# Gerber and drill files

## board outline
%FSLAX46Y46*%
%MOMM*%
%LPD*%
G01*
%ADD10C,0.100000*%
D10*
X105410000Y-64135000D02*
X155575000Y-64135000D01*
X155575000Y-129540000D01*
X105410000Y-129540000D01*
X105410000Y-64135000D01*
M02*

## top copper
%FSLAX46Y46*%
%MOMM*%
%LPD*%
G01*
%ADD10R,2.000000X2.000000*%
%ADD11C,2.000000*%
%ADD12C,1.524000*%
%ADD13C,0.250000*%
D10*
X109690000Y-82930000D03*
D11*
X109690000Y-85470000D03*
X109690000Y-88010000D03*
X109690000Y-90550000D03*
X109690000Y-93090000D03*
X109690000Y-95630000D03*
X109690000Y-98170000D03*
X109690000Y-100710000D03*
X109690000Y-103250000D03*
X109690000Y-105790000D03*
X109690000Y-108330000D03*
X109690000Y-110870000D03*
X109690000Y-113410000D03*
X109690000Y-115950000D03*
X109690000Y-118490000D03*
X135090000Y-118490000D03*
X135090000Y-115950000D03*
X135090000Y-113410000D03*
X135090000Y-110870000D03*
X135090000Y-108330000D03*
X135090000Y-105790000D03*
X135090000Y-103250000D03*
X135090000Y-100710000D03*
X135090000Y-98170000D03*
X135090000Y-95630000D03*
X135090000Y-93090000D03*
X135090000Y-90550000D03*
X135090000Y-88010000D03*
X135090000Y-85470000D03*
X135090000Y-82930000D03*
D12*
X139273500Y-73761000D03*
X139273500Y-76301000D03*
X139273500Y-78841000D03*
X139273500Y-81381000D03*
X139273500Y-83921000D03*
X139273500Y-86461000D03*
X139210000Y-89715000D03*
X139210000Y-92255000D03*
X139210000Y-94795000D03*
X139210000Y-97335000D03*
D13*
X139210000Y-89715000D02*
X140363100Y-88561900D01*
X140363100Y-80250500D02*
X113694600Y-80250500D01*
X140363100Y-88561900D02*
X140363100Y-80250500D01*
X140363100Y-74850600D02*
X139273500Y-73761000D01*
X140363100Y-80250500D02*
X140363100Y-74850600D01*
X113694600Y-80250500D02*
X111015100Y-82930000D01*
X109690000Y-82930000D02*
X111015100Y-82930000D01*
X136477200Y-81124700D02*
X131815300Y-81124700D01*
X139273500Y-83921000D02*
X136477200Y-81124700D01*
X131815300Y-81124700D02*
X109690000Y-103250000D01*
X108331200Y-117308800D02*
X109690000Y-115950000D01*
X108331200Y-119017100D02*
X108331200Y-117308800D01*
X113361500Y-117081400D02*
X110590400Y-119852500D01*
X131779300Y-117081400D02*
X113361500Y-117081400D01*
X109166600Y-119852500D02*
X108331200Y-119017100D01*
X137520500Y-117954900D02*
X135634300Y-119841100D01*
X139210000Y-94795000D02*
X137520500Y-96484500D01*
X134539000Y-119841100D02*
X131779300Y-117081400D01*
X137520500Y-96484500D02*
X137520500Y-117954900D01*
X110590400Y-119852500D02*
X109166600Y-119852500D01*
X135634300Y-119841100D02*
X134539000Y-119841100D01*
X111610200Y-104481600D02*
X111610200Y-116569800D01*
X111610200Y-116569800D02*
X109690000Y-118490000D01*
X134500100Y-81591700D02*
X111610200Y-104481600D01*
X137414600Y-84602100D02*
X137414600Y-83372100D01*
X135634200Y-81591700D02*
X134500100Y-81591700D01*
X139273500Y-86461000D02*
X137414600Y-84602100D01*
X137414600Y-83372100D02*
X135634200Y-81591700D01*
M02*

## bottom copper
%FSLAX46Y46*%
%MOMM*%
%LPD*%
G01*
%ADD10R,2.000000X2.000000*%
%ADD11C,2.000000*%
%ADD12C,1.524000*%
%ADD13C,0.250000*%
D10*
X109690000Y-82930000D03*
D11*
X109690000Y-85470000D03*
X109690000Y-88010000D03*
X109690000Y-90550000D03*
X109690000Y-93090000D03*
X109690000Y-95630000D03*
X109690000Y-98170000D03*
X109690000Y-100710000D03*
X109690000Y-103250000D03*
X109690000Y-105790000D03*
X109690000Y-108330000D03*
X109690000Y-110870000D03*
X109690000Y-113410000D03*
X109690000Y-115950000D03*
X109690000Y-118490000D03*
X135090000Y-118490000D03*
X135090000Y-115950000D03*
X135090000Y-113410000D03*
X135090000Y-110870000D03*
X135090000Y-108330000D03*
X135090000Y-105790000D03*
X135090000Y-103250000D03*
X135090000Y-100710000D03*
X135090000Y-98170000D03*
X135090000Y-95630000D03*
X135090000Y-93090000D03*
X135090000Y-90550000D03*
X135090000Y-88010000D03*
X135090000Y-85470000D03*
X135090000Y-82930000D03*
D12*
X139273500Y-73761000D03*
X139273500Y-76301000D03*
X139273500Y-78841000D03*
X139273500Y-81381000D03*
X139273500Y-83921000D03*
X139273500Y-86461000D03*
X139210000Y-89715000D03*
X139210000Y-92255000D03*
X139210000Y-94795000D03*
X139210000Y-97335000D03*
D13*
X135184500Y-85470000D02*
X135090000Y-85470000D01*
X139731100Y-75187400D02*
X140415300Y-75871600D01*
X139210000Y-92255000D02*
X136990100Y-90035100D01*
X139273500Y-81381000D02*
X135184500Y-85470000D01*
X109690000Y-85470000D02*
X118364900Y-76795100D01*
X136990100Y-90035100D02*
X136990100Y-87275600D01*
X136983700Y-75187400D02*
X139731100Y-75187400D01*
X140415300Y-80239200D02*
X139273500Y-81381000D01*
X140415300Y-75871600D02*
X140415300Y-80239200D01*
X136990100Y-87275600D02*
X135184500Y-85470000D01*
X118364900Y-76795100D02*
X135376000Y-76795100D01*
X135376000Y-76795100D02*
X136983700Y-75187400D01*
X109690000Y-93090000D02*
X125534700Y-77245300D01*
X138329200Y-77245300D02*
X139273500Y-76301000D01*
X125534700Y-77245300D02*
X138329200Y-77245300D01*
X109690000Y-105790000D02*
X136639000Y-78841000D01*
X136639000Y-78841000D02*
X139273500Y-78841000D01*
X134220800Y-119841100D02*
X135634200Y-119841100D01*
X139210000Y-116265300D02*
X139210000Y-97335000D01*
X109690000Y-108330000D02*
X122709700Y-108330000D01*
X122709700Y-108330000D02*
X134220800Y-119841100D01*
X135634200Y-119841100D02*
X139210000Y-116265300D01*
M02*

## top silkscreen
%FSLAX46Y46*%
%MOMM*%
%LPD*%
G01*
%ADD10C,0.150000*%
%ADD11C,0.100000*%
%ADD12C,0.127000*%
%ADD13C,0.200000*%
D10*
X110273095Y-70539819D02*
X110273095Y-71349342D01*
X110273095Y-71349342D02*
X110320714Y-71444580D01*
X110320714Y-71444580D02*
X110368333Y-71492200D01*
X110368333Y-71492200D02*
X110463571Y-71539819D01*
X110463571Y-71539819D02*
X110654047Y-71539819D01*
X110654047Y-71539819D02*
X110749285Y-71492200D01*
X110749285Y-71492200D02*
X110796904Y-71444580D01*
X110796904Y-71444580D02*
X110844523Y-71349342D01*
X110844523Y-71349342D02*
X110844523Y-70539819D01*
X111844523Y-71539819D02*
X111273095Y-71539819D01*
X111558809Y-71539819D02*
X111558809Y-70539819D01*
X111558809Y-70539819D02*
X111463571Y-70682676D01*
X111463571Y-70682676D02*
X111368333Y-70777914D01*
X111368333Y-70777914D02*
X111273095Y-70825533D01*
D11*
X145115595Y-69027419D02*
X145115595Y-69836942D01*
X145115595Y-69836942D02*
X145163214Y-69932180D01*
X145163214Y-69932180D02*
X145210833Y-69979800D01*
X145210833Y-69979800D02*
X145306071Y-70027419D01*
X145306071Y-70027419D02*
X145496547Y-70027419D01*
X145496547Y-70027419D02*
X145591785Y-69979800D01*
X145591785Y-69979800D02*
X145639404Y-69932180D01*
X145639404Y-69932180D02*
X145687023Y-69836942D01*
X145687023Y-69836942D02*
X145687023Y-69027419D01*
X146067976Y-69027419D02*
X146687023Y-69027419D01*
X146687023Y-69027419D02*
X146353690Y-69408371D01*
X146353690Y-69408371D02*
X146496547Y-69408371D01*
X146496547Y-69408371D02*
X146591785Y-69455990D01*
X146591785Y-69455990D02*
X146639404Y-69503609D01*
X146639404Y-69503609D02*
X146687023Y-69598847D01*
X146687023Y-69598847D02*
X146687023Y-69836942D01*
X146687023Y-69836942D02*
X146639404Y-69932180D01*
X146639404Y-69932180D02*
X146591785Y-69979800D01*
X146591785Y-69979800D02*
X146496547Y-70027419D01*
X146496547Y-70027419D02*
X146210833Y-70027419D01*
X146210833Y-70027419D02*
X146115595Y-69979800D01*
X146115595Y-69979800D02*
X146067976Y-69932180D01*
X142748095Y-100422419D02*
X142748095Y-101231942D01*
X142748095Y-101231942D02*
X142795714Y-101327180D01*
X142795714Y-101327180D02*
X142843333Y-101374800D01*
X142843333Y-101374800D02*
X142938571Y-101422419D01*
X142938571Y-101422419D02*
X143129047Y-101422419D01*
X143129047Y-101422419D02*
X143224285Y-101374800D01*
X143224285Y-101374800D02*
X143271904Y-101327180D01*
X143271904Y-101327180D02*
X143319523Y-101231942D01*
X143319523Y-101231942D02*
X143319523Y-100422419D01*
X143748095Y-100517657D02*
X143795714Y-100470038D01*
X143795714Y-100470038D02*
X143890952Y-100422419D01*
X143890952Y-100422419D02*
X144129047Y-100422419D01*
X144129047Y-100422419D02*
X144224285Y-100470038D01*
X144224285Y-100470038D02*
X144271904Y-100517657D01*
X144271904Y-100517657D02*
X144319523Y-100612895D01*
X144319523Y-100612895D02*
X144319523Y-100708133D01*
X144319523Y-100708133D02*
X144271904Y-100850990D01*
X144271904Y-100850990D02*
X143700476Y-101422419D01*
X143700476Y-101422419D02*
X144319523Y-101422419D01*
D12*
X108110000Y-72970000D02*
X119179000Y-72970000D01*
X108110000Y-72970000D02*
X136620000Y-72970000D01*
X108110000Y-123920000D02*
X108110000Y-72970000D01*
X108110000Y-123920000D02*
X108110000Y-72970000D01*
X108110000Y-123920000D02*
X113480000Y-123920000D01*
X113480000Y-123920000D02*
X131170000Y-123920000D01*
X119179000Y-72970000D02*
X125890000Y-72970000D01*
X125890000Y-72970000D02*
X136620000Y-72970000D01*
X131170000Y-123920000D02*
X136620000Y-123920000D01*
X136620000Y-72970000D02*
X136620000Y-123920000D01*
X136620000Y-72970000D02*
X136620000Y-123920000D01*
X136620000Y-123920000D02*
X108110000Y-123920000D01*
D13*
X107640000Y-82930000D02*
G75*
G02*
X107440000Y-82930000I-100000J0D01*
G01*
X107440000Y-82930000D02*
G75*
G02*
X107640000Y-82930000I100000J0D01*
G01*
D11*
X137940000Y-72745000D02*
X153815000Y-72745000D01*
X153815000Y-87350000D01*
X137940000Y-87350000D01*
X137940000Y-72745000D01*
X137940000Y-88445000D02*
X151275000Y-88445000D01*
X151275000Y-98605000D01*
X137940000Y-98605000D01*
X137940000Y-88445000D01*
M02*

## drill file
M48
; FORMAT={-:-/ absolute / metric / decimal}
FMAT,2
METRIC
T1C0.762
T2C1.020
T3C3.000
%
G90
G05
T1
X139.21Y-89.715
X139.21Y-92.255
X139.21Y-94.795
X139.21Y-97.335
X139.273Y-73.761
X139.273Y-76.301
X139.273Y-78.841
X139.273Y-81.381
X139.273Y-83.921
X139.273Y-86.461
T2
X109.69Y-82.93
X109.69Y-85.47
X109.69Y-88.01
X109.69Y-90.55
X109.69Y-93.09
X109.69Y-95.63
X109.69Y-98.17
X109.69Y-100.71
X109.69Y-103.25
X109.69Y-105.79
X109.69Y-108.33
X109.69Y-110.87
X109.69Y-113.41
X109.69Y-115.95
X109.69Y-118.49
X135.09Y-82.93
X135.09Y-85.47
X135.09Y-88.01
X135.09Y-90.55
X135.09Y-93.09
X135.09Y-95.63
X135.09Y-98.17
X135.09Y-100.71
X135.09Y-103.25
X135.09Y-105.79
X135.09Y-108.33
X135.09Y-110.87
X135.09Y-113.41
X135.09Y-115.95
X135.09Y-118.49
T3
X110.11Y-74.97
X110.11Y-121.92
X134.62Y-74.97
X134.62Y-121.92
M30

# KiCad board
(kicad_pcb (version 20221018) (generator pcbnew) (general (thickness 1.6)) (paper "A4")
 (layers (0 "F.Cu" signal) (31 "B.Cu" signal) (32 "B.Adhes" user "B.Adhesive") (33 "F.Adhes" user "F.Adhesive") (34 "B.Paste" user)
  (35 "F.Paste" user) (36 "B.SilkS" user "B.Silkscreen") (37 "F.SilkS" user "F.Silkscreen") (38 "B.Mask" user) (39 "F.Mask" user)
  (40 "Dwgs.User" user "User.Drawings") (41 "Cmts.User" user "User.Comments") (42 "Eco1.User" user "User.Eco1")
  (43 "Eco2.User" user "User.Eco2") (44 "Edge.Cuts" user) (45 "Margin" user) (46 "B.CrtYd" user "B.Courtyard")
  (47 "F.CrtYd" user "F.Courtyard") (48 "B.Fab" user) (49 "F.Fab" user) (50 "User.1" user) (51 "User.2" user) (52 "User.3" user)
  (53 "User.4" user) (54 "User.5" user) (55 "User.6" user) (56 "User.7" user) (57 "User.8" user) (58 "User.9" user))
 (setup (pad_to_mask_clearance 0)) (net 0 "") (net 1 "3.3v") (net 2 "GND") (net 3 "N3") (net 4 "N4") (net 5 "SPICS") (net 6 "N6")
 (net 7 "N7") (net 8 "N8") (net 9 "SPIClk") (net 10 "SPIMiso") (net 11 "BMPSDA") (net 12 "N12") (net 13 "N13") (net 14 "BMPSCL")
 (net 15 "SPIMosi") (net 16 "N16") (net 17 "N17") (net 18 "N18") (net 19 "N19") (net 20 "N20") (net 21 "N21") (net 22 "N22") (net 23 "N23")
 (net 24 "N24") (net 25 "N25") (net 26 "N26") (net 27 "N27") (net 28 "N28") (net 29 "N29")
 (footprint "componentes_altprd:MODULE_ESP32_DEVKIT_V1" (layer "F.Cu") (at 122.39 98.445)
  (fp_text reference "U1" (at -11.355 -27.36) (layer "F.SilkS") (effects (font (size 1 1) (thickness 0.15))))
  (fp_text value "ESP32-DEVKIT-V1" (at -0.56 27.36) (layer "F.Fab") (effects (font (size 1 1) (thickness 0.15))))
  (fp_line (start -14.28 -25.475) (end -3.211 -25.475) (stroke (width 0.127) (type solid)) (layer "F.SilkS"))
  (fp_line (start -14.28 -25.475) (end 14.23 -25.475) (stroke (width 0.127) (type solid)) (layer "F.SilkS"))
  (fp_line (start -14.28 25.475) (end -14.28 -25.475) (stroke (width 0.127) (type solid)) (layer "F.SilkS"))
  (fp_line (start -14.28 25.475) (end -14.28 -25.475) (stroke (width 0.127) (type solid)) (layer "F.SilkS"))
  (fp_line (start -14.28 25.475) (end -8.91 25.475) (stroke (width 0.127) (type solid)) (layer "F.SilkS"))
  (fp_line (start -8.91 25.475) (end 8.78 25.475) (stroke (width 0.127) (type solid)) (layer "F.SilkS"))
  (fp_line (start -3.211 -25.475) (end 3.5 -25.475) (stroke (width 0.127) (type solid)) (layer "F.SilkS"))
  (fp_line (start 3.5 -25.475) (end 14.23 -25.475) (stroke (width 0.127) (type solid)) (layer "F.SilkS"))
  (fp_line (start 8.78 25.475) (end 14.23 25.475) (stroke (width 0.127) (type solid)) (layer "F.SilkS"))
  (fp_line (start 14.23 -25.475) (end 14.23 25.475) (stroke (width 0.127) (type solid)) (layer "F.SilkS"))
  (fp_line (start 14.23 -25.475) (end 14.23 25.475) (stroke (width 0.127) (type solid)) (layer "F.SilkS"))
  (fp_line (start 14.23 25.475) (end -14.28 25.475) (stroke (width 0.127) (type solid)) (layer "F.SilkS"))
  (fp_circle (center -14.85 -15.515) (end -14.75 -15.515) (stroke (width 0.2) (type solid)) (fill none) (layer "F.SilkS"))
  (pad "" np_thru_hole circle (at -12.28 -23.475) (size 3 3) (drill 3) (layers "*.Cu" "*.Mask"))
  (pad "" np_thru_hole circle (at -12.28 23.475) (size 3 3) (drill 3) (layers "*.Cu" "*.Mask"))
  (pad "" np_thru_hole circle (at 12.23 -23.475) (size 3 3) (drill 3) (layers "*.Cu" "*.Mask"))
  (pad "" np_thru_hole circle (at 12.23 23.475) (size 3 3) (drill 3) (layers "*.Cu" "*.Mask"))
  (pad "1" thru_hole rect (at -12.7 -15.515) (size 2 2) (drill 1.02) (layers "*.Cu" "*.Mask") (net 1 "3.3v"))
  (pad "2" thru_hole circle (at -12.7 -12.975) (size 2 2) (drill 1.02) (layers "*.Cu" "*.Mask") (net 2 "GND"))
  (pad "3" thru_hole circle (at -12.7 -10.435) (size 2 2) (drill 1.02) (layers "*.Cu" "*.Mask") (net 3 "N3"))
  (pad "4" thru_hole circle (at -12.7 -7.895) (size 2 2) (drill 1.02) (layers "*.Cu" "*.Mask") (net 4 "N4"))
  (pad "5" thru_hole circle (at -12.7 -5.355) (size 2 2) (drill 1.02) (layers "*.Cu" "*.Mask") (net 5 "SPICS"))
  (pad "6" thru_hole circle (at -12.7 -2.815) (size 2 2) (drill 1.02) (layers "*.Cu" "*.Mask") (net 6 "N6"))
  (pad "7" thru_hole circle (at -12.7 -0.275) (size 2 2) (drill 1.02) (layers "*.Cu" "*.Mask") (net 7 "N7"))
  (pad "8" thru_hole circle (at -12.7 2.265) (size 2 2) (drill 1.02) (layers "*.Cu" "*.Mask") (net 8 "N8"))
  (pad "9" thru_hole circle (at -12.7 4.805) (size 2 2) (drill 1.02) (layers "*.Cu" "*.Mask") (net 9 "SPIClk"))
  (pad "10" thru_hole circle (at -12.7 7.345) (size 2 2) (drill 1.02) (layers "*.Cu" "*.Mask") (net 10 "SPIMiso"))
  (pad "11" thru_hole circle (at -12.7 9.885) (size 2 2) (drill 1.02) (layers "*.Cu" "*.Mask") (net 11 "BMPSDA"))
  (pad "12" thru_hole circle (at -12.7 12.425) (size 2 2) (drill 1.02) (layers "*.Cu" "*.Mask") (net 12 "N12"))
  (pad "13" thru_hole circle (at -12.7 14.965) (size 2 2) (drill 1.02) (layers "*.Cu" "*.Mask") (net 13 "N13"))
  (pad "14" thru_hole circle (at -12.7 17.505) (size 2 2) (drill 1.02) (layers "*.Cu" "*.Mask") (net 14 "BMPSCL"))
  (pad "15" thru_hole circle (at -12.7 20.045) (size 2 2) (drill 1.02) (layers "*.Cu" "*.Mask") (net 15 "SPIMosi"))
  (pad "16" thru_hole circle (at 12.7 20.045) (size 2 2) (drill 1.02) (layers "*.Cu" "*.Mask") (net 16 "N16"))
  (pad "17" thru_hole circle (at 12.7 17.505) (size 2 2) (drill 1.02) (layers "*.Cu" "*.Mask") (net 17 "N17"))
  (pad "18" thru_hole circle (at 12.7 14.965) (size 2 2) (drill 1.02) (layers "*.Cu" "*.Mask") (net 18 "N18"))
  (pad "19" thru_hole circle (at 12.7 12.425) (size 2 2) (drill 1.02) (layers "*.Cu" "*.Mask") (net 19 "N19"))
  (pad "20" thru_hole circle (at 12.7 9.885) (size 2 2) (drill 1.02) (layers "*.Cu" "*.Mask") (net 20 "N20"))
  (pad "21" thru_hole circle (at 12.7 7.345) (size 2 2) (drill 1.02) (layers "*.Cu" "*.Mask") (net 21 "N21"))
  (pad "22" thru_hole circle (at 12.7 4.805) (size 2 2) (drill 1.02) (layers "*.Cu" "*.Mask") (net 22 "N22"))
  (pad "23" thru_hole circle (at 12.7 2.265) (size 2 2) (drill 1.02) (layers "*.Cu" "*.Mask") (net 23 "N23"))
  (pad "24" thru_hole circle (at 12.7 -0.275) (size 2 2) (drill 1.02) (layers "*.Cu" "*.Mask") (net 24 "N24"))
  (pad "25" thru_hole circle (at 12.7 -2.815) (size 2 2) (drill 1.02) (layers "*.Cu" "*.Mask") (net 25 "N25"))
  (pad "26" thru_hole circle (at 12.7 -5.355) (size 2 2) (drill 1.02) (layers "*.Cu" "*.Mask") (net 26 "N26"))
  (pad "27" thru_hole circle (at 12.7 -7.895) (size 2 2) (drill 1.02) (layers "*.Cu" "*.Mask") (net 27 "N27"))
  (pad "28" thru_hole circle (at 12.7 -10.435) (size 2 2) (drill 1.02) (layers "*.Cu" "*.Mask") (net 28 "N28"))
  (pad "29" thru_hole circle (at 12.7 -12.975) (size 2 2) (drill 1.02) (layers "*.Cu" "*.Mask") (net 2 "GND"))
  (pad "30" thru_hole circle (at 12.7 -15.515) (size 2 2) (drill 1.02) (layers "*.Cu" "*.Mask") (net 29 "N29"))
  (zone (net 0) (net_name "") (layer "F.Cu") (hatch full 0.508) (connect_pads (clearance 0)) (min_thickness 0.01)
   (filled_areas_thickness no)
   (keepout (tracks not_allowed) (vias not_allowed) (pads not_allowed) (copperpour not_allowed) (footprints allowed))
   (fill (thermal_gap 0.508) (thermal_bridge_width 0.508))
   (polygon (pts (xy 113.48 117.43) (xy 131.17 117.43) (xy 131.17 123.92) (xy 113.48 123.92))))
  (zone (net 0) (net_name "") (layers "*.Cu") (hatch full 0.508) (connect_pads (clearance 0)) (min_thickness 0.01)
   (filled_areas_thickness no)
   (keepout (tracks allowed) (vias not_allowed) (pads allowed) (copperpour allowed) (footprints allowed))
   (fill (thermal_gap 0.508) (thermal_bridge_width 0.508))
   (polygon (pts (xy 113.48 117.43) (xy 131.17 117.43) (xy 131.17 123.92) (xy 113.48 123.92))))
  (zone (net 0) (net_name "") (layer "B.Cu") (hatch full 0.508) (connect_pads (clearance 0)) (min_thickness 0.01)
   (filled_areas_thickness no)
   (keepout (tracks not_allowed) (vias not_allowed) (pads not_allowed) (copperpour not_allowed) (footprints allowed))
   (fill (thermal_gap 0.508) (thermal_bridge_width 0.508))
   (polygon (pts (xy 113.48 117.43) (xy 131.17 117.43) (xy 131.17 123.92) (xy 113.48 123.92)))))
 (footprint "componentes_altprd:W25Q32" (layer "F.Cu") (at 146.195 79.73)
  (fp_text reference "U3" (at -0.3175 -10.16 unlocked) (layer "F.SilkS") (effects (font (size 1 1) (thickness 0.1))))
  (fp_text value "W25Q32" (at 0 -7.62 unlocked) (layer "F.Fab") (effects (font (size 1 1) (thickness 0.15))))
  (fp_rect (start -8.255 -6.985) (end 7.62 7.62) (stroke (width 0.1) (type default)) (fill none) (layer "F.SilkS"))
  (pad "1" thru_hole circle (at -6.9215 -5.969) (size 1.524 1.524) (drill 0.762) (layers "*.Cu" "*.Mask") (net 1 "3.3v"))
  (pad "2" thru_hole circle (at -6.9215 -3.429) (size 1.524 1.524) (drill 0.762) (layers "*.Cu" "*.Mask") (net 5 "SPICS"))
  (pad "3" thru_hole circle (at -6.9215 -0.889) (size 1.524 1.524) (drill 0.762) (layers "*.Cu" "*.Mask") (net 10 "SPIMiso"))
  (pad "4" thru_hole circle (at -6.9215 1.651) (size 1.524 1.524) (drill 0.762) (layers "*.Cu" "*.Mask") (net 2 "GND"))
  (pad "5" thru_hole circle (at -6.9215 4.191) (size 1.524 1.524) (drill 0.762) (layers "*.Cu" "*.Mask") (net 9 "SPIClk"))
  (pad "6" thru_hole circle (at -6.9215 6.731) (size 1.524 1.524) (drill 0.762) (layers "*.Cu" "*.Mask") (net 15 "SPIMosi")))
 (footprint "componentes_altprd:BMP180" (layer "F.Cu") (at 143.655 94.795)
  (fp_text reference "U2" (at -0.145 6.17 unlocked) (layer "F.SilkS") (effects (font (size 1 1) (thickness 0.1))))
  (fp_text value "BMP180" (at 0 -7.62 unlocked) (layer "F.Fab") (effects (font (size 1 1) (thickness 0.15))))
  (fp_rect (start -5.715 -6.35) (end 7.62 3.81) (stroke (width 0.1) (type default)) (fill none) (layer "F.SilkS"))
  (pad "1" thru_hole circle (at -4.445 -5.08) (size 1.524 1.524) (drill 0.762) (layers "*.Cu" "*.Mask") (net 1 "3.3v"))
  (pad "2" thru_hole circle (at -4.445 -2.54) (size 1.524 1.524) (drill 0.762) (layers "*.Cu" "*.Mask") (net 2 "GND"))
  (pad "3" thru_hole circle (at -4.445 0) (size 1.524 1.524) (drill 0.762) (layers "*.Cu" "*.Mask") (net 14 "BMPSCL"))
  (pad "4" thru_hole circle (at -4.445 2.54) (size 1.524 1.524) (drill 0.762) (layers "*.Cu" "*.Mask") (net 11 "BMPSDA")))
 (gr_rect (start 105.41 64.135) (end 155.575 129.54) (stroke (width 0.1) (type default)) (fill none) (layer "Edge.Cuts"))
 (segment (start 139.21 89.715) (end 140.3631 88.5619) (width 0.25) (layer "F.Cu") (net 1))
 (segment (start 140.3631 80.2505) (end 113.6946 80.2505) (width 0.25) (layer "F.Cu") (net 1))
 (segment (start 140.3631 88.5619) (end 140.3631 80.2505) (width 0.25) (layer "F.Cu") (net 1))
 (segment (start 140.3631 74.8506) (end 139.2735 73.761) (width 0.25) (layer "F.Cu") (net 1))
 (segment (start 140.3631 80.2505) (end 140.3631 74.8506) (width 0.25) (layer "F.Cu") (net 1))
 (segment (start 113.6946 80.2505) (end 111.0151 82.93) (width 0.25) (layer "F.Cu") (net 1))
 (segment (start 109.69 82.93) (end 111.0151 82.93) (width 0.25) (layer "F.Cu") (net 1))
 (segment (start 135.1845 85.47) (end 135.09 85.47) (width 0.25) (layer "B.Cu") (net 2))
 (segment (start 139.7311 75.1874) (end 140.4153 75.8716) (width 0.25) (layer "B.Cu") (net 2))
 (segment (start 139.21 92.255) (end 136.9901 90.0351) (width 0.25) (layer "B.Cu") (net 2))
 (segment (start 139.2735 81.381) (end 135.1845 85.47) (width 0.25) (layer "B.Cu") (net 2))
 (segment (start 109.69 85.47) (end 118.3649 76.7951) (width 0.25) (layer "B.Cu") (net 2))
 (segment (start 136.9901 90.0351) (end 136.9901 87.2756) (width 0.25) (layer "B.Cu") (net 2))
 (segment (start 136.9837 75.1874) (end 139.7311 75.1874) (width 0.25) (layer "B.Cu") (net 2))
 (segment (start 140.4153 80.2392) (end 139.2735 81.381) (width 0.25) (layer "B.Cu") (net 2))
 (segment (start 140.4153 75.8716) (end 140.4153 80.2392) (width 0.25) (layer "B.Cu") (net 2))
 (segment (start 136.9901 87.2756) (end 135.1845 85.47) (width 0.25) (layer "B.Cu") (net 2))
 (segment (start 118.3649 76.7951) (end 135.376 76.7951) (width 0.25) (layer "B.Cu") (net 2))
 (segment (start 135.376 76.7951) (end 136.9837 75.1874) (width 0.25) (layer "B.Cu") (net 2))
 (segment (start 109.69 93.09) (end 125.5347 77.2453) (width 0.25) (layer "B.Cu") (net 5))
 (segment (start 138.3292 77.2453) (end 139.2735 76.301) (width 0.25) (layer "B.Cu") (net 5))
 (segment (start 125.5347 77.2453) (end 138.3292 77.2453) (width 0.25) (layer "B.Cu") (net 5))
 (segment (start 136.4772 81.1247) (end 131.8153 81.1247) (width 0.25) (layer "F.Cu") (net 9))
 (segment (start 139.2735 83.921) (end 136.4772 81.1247) (width 0.25) (layer "F.Cu") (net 9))
 (segment (start 131.8153 81.1247) (end 109.69 103.25) (width 0.25) (layer "F.Cu") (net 9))
 (segment (start 109.69 105.79) (end 136.639 78.841) (width 0.25) (layer "B.Cu") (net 10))
 (segment (start 136.639 78.841) (end 139.2735 78.841) (width 0.25) (layer "B.Cu") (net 10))
 (segment (start 134.2208 119.8411) (end 135.6342 119.8411) (width 0.25) (layer "B.Cu") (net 11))
 (segment (start 139.21 116.2653) (end 139.21 97.335) (width 0.25) (layer "B.Cu") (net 11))
 (segment (start 109.69 108.33) (end 122.7097 108.33) (width 0.25) (layer "B.Cu") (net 11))
 (segment (start 122.7097 108.33) (end 134.2208 119.8411) (width 0.25) (layer "B.Cu") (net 11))
 (segment (start 135.6342 119.8411) (end 139.21 116.2653) (width 0.25) (layer "B.Cu") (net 11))
 (segment (start 108.3312 117.3088) (end 109.69 115.95) (width 0.25) (layer "F.Cu") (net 14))
 (segment (start 108.3312 119.0171) (end 108.3312 117.3088) (width 0.25) (layer "F.Cu") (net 14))
 (segment (start 113.3615 117.0814) (end 110.5904 119.8525) (width 0.25) (layer "F.Cu") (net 14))
 (segment (start 131.7793 117.0814) (end 113.3615 117.0814) (width 0.25) (layer "F.Cu") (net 14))
 (segment (start 109.1666 119.8525) (end 108.3312 119.0171) (width 0.25) (layer "F.Cu") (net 14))
 (segment (start 137.5205 117.9549) (end 135.6343 119.8411) (width 0.25) (layer "F.Cu") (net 14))
 (segment (start 139.21 94.795) (end 137.5205 96.4845) (width 0.25) (layer "F.Cu") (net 14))
 (segment (start 134.539 119.8411) (end 131.7793 117.0814) (width 0.25) (layer "F.Cu") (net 14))
 (segment (start 137.5205 96.4845) (end 137.5205 117.9549) (width 0.25) (layer "F.Cu") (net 14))
 (segment (start 110.5904 119.8525) (end 109.1666 119.8525) (width 0.25) (layer "F.Cu") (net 14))
 (segment (start 135.6343 119.8411) (end 134.539 119.8411) (width 0.25) (layer "F.Cu") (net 14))
 (segment (start 111.6102 104.4816) (end 111.6102 116.5698) (width 0.25) (layer "F.Cu") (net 15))
 (segment (start 111.6102 116.5698) (end 109.69 118.49) (width 0.25) (layer "F.Cu") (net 15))
 (segment (start 134.5001 81.5917) (end 111.6102 104.4816) (width 0.25) (layer "F.Cu") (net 15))
 (segment (start 137.4146 84.6021) (end 137.4146 83.3721) (width 0.25) (layer "F.Cu") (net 15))
 (segment (start 135.6342 81.5917) (end 134.5001 81.5917) (width 0.25) (layer "F.Cu") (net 15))
 (segment (start 139.2735 86.461) (end 137.4146 84.6021) (width 0.25) (layer "F.Cu") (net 15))
 (segment (start 137.4146 83.3721) (end 135.6342 81.5917) (width 0.25) (layer "F.Cu") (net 15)))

